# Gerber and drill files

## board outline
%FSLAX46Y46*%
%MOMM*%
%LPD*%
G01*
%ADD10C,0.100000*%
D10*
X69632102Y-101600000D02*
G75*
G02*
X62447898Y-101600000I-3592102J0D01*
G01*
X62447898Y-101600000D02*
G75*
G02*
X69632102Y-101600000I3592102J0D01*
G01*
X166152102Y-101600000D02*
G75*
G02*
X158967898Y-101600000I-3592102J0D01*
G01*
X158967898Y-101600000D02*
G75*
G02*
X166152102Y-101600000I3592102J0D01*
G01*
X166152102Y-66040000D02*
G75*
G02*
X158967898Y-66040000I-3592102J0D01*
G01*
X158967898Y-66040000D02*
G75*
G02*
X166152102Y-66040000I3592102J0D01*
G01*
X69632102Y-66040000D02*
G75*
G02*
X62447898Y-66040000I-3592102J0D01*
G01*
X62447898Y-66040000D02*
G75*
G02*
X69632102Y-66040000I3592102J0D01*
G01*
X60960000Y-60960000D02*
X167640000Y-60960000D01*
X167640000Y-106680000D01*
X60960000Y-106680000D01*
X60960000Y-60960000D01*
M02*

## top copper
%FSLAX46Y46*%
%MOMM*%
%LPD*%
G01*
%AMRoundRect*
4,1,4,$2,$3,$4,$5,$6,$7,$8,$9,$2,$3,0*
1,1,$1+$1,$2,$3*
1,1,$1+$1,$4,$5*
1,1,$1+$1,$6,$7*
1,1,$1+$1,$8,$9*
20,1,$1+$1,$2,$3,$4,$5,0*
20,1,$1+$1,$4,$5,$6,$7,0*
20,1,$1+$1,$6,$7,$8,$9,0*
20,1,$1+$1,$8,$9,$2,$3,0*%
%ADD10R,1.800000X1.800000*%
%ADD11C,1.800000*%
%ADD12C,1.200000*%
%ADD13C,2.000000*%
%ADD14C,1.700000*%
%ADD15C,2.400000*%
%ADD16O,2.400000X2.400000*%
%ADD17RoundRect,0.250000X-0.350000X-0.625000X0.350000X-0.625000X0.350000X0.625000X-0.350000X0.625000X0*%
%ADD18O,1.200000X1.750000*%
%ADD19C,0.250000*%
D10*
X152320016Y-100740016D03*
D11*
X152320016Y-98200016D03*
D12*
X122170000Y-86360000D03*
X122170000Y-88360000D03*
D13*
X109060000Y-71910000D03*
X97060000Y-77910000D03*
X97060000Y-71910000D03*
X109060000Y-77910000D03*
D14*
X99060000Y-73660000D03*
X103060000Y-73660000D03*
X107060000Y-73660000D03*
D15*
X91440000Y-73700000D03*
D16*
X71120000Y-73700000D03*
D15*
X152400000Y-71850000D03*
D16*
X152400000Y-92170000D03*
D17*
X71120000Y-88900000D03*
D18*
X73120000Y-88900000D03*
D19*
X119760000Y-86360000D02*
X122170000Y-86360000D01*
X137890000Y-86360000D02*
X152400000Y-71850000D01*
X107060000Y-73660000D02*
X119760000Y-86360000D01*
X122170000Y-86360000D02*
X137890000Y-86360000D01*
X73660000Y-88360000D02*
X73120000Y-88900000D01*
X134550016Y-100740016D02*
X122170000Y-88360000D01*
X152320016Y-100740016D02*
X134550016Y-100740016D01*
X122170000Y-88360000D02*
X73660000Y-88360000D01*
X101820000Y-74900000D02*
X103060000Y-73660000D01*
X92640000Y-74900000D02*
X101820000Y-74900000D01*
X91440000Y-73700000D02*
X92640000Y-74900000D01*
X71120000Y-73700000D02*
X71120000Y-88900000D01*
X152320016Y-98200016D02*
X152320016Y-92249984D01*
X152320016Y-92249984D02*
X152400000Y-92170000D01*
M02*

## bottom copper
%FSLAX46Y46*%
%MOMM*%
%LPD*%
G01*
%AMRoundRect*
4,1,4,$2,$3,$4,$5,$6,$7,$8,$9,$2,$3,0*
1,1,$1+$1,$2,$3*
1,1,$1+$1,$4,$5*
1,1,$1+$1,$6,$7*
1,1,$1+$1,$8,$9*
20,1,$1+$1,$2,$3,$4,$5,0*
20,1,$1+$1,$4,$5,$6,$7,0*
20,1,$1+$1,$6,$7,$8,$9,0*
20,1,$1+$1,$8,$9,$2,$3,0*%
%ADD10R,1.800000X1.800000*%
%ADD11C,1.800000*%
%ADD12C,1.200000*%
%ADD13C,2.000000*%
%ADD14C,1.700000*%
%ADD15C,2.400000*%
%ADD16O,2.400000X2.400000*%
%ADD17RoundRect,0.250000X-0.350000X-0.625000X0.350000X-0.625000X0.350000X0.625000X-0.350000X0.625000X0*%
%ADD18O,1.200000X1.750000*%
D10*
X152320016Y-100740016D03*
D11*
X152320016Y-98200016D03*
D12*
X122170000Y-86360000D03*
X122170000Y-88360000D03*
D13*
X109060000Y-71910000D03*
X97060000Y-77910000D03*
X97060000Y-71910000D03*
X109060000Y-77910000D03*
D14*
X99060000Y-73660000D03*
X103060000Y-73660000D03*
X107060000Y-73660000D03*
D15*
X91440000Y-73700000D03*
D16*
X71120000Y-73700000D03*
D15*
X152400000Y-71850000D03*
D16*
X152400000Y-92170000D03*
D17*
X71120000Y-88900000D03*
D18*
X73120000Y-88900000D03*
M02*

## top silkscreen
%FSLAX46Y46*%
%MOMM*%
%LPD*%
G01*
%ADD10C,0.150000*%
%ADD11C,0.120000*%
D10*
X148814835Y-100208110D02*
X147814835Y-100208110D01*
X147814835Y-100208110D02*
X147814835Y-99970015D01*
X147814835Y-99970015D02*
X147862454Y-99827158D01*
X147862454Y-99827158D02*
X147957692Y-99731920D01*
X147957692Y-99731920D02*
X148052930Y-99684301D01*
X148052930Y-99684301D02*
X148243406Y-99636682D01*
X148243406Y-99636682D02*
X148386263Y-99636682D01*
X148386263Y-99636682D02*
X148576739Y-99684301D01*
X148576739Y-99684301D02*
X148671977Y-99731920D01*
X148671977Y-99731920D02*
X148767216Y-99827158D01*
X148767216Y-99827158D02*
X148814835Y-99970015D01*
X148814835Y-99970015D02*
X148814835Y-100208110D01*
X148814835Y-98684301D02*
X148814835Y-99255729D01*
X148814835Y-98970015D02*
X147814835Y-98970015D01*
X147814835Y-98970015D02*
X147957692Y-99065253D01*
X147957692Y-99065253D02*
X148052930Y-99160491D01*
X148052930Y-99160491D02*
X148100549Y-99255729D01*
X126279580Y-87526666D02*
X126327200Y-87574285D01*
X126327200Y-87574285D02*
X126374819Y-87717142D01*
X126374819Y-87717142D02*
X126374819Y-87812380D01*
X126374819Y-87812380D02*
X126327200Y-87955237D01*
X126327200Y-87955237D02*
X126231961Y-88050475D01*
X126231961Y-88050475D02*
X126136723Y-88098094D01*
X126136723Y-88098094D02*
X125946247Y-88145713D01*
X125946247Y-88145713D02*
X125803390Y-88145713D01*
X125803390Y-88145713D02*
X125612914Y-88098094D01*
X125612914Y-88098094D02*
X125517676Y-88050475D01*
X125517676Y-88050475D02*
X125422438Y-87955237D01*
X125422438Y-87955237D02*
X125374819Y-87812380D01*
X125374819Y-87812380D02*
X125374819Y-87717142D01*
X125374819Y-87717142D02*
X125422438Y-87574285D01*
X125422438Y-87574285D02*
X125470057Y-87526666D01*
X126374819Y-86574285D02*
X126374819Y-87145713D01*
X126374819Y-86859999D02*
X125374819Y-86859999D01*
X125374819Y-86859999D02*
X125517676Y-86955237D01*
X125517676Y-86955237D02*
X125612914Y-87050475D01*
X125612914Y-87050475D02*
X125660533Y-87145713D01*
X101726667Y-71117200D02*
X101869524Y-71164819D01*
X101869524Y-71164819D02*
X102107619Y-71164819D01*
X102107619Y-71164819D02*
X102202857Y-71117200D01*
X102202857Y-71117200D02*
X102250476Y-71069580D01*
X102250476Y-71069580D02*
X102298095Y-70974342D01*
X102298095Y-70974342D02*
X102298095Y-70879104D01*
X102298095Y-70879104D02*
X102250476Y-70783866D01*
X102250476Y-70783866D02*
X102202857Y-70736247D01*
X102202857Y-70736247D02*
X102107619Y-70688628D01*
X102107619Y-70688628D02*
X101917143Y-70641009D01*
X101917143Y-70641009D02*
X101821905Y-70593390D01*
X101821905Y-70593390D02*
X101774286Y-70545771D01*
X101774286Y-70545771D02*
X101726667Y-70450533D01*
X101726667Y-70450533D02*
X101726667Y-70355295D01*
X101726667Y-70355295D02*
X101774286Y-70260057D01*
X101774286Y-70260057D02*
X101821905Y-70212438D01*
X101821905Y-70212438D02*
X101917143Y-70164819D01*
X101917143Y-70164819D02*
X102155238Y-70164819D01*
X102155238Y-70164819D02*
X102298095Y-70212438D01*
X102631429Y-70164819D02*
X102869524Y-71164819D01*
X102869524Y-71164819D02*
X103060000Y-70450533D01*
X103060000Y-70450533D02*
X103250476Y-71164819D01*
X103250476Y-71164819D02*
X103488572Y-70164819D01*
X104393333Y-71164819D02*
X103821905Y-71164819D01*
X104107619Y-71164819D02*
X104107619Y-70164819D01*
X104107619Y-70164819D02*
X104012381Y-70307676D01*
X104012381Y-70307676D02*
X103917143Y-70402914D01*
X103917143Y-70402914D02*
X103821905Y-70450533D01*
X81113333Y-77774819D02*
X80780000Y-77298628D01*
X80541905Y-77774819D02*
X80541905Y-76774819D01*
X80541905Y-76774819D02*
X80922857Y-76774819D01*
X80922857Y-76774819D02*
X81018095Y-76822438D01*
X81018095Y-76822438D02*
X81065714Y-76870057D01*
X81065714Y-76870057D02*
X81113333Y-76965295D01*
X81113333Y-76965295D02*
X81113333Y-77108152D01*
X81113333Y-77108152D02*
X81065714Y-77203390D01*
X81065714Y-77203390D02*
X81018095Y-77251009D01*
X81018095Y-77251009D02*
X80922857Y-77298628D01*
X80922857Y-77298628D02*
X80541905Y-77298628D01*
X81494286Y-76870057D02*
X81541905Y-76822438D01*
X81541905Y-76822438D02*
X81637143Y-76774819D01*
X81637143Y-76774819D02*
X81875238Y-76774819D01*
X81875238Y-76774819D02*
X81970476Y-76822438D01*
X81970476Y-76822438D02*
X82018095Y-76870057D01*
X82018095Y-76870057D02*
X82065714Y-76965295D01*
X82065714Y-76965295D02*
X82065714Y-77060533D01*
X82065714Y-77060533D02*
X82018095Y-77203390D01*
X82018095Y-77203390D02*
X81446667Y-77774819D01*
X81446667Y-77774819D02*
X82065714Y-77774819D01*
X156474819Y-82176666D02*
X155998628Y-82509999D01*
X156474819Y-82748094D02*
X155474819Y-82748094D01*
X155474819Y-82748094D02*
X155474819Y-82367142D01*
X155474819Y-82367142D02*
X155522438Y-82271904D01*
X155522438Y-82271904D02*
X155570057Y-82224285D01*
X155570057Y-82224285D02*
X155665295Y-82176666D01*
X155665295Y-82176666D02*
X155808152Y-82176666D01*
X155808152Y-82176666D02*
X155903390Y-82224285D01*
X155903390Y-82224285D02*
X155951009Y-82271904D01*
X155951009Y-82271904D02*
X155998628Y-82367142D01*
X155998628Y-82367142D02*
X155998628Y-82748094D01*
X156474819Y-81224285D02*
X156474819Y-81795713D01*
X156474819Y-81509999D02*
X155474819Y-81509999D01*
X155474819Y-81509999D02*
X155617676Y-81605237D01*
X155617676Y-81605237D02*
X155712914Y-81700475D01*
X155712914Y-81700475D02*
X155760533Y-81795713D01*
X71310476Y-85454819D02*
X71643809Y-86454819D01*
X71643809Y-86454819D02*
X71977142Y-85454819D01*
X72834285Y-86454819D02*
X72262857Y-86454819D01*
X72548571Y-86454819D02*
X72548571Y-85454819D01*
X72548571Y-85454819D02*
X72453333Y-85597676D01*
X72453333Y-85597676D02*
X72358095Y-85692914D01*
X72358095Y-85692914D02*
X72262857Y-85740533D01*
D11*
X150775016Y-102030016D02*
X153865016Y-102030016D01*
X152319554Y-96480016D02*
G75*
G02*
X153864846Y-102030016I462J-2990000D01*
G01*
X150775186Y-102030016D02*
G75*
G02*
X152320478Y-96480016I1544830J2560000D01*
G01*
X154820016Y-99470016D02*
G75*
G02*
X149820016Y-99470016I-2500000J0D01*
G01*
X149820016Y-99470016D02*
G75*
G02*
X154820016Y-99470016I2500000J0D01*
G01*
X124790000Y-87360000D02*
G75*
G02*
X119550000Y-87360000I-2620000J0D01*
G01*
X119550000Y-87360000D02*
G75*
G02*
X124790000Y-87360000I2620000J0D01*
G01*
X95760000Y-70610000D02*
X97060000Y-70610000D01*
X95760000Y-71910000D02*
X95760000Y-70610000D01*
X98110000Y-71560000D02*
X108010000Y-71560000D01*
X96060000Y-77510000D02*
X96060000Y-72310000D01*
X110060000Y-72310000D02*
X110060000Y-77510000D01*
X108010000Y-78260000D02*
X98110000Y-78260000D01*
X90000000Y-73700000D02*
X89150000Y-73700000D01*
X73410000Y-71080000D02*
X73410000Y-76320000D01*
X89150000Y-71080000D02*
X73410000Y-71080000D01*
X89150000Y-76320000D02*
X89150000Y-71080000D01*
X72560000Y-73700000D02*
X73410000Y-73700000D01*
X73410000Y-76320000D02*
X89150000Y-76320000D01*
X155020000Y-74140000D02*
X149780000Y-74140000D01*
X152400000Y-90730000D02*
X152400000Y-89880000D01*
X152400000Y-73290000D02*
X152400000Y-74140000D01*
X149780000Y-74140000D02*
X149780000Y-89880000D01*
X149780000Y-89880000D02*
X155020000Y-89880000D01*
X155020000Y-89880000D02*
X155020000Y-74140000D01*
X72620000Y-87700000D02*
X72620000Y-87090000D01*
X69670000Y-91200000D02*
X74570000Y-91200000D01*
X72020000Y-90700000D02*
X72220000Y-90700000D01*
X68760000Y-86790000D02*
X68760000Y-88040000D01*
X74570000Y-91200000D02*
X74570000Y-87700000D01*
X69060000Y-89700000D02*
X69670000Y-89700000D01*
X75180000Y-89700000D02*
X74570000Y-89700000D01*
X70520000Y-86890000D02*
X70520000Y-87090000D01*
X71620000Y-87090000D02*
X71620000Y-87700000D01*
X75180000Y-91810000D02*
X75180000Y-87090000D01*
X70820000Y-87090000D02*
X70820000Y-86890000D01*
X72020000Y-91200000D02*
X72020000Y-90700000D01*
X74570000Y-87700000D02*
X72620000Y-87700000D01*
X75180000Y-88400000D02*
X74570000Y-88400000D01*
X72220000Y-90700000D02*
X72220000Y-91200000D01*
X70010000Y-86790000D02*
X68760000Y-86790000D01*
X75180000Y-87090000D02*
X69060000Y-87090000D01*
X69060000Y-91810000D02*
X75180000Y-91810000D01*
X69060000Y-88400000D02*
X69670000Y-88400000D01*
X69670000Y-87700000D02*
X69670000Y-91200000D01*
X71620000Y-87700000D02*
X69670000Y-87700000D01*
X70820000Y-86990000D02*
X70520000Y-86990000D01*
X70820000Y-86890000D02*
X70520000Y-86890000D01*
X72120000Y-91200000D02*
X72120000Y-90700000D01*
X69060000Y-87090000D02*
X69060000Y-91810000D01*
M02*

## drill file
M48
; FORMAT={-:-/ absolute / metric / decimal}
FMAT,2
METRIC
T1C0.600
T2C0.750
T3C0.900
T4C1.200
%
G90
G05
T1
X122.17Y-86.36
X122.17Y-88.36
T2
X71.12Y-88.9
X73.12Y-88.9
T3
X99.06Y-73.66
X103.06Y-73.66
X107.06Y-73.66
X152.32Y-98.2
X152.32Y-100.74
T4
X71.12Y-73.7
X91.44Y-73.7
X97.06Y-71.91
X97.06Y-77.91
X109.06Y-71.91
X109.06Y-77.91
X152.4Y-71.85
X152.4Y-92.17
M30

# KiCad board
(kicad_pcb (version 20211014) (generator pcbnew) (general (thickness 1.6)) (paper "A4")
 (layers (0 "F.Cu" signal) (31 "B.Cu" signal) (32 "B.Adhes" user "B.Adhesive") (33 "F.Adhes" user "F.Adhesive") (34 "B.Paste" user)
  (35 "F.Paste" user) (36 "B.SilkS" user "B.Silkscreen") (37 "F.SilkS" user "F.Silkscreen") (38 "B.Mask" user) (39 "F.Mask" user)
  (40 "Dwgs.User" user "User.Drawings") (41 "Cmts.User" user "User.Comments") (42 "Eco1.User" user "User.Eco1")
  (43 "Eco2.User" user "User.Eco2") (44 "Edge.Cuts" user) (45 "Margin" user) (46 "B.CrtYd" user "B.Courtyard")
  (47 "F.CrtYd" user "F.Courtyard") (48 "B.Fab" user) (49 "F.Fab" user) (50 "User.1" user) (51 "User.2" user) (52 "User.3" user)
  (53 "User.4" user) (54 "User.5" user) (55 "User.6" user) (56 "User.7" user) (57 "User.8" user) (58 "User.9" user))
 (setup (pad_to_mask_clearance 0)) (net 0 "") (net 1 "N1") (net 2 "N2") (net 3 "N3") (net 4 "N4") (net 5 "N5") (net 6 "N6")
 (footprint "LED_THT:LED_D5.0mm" (layer "F.Cu") (at 152.320016 100.740016 90)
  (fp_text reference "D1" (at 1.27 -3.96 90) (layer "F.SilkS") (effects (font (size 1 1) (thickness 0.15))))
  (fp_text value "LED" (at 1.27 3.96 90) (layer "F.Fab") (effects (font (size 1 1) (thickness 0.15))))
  (fp_line (start -1.29 -1.545) (end -1.29 1.545) (layer "F.SilkS") (width 0.12))
  (fp_arc (start 4.26 -0.000462) (mid 2.072002 2.880433) (end -1.29 1.54483) (layer "F.SilkS") (width 0.12))
  (fp_arc (start -1.29 -1.54483) (mid 2.072002 -2.880433) (end 4.26 0.000462) (layer "F.SilkS") (width 0.12))
  (fp_circle (center 1.27 0) (end 3.77 0) (layer "F.SilkS") (width 0.12) (fill none))
  (pad "1" thru_hole rect (at 0 0 90) (size 1.8 1.8) (drill 0.9) (layers *.Cu *.Mask) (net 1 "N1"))
  (pad "2" thru_hole circle (at 2.54 0 90) (size 1.8 1.8) (drill 0.9) (layers *.Cu *.Mask) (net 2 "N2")))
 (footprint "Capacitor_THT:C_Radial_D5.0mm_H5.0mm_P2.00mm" (layer "F.Cu") (at 122.17 86.36 -90)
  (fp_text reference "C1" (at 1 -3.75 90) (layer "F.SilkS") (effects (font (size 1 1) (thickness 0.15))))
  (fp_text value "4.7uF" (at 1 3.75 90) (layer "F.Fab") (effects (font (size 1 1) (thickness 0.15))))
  (fp_circle (center 1 0) (end 3.62 0) (layer "F.SilkS") (width 0.12) (fill none))
  (pad "1" thru_hole circle (at 0 0 270) (size 1.2 1.2) (drill 0.6) (layers *.Cu *.Mask) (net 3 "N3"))
  (pad "2" thru_hole circle (at 2 0 270) (size 1.2 1.2) (drill 0.6) (layers *.Cu *.Mask) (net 1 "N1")))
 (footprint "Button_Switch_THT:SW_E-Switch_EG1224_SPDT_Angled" (layer "F.Cu") (at 99.06 73.66)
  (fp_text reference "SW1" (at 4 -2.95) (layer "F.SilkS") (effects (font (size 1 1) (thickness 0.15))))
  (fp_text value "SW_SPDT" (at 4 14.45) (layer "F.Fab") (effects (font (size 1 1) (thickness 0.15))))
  (fp_line (start -3.3 -3.05) (end -2 -3.05) (layer "F.SilkS") (width 0.12))
  (fp_line (start -3.3 -1.75) (end -3.3 -3.05) (layer "F.SilkS") (width 0.12))
  (fp_line (start -0.95 -2.1) (end 8.95 -2.1) (layer "F.SilkS") (width 0.12))
  (fp_line (start -3 3.85) (end -3 -1.35) (layer "F.SilkS") (width 0.12))
  (fp_line (start 11 -1.35) (end 11 3.85) (layer "F.SilkS") (width 0.12))
  (fp_line (start 8.95 4.6) (end -0.95 4.6) (layer "F.SilkS") (width 0.12))
  (pad "" thru_hole circle (at 10 -1.75) (size 2 2) (drill 1.2) (layers *.Cu *.Mask))
  (pad "" thru_hole circle (at -2 4.25) (size 2 2) (drill 1.2) (layers *.Cu *.Mask))
  (pad "" thru_hole circle (at -2 -1.75) (size 2 2) (drill 1.2) (layers *.Cu *.Mask))
  (pad "" thru_hole circle (at 10 4.25) (size 2 2) (drill 1.2) (layers *.Cu *.Mask))
  (pad "1" thru_hole circle (at 0 0) (size 1.7 1.7) (drill 0.9) (layers *.Cu *.Mask) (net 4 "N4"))
  (pad "2" thru_hole circle (at 4 0) (size 1.7 1.7) (drill 0.9) (layers *.Cu *.Mask) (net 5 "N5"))
  (pad "3" thru_hole circle (at 8 0) (size 1.7 1.7) (drill 0.9) (layers *.Cu *.Mask) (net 3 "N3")))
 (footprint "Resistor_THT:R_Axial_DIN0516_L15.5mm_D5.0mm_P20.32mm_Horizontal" (layer "F.Cu") (at 91.44 73.7 180)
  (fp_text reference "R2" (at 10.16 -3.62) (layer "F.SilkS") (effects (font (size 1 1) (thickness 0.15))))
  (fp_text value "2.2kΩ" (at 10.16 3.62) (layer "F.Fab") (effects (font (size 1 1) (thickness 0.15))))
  (fp_line (start 1.44 0) (end 2.29 0) (layer "F.SilkS") (width 0.12))
  (fp_line (start 18.03 2.62) (end 18.03 -2.62) (layer "F.SilkS") (width 0.12))
  (fp_line (start 2.29 2.62) (end 18.03 2.62) (layer "F.SilkS") (width 0.12))
  (fp_line (start 2.29 -2.62) (end 2.29 2.62) (layer "F.SilkS") (width 0.12))
  (fp_line (start 18.88 0) (end 18.03 0) (layer "F.SilkS") (width 0.12))
  (fp_line (start 18.03 -2.62) (end 2.29 -2.62) (layer "F.SilkS") (width 0.12))
  (pad "1" thru_hole circle (at 0 0 180) (size 2.4 2.4) (drill 1.2) (layers *.Cu *.Mask) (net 5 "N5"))
  (pad "2" thru_hole oval (at 20.32 0 180) (size 2.4 2.4) (drill 1.2) (layers *.Cu *.Mask) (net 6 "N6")))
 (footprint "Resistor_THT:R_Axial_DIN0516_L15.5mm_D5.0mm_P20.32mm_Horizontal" (layer "F.Cu") (at 152.4 71.85 -90)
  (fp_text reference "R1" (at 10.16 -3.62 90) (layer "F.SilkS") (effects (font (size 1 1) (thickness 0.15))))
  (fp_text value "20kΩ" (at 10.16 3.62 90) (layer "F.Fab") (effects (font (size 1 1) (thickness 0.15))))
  (fp_line (start 2.29 -2.62) (end 2.29 2.62) (layer "F.SilkS") (width 0.12))
  (fp_line (start 18.88 0) (end 18.03 0) (layer "F.SilkS") (width 0.12))
  (fp_line (start 1.44 0) (end 2.29 0) (layer "F.SilkS") (width 0.12))
  (fp_line (start 2.29 2.62) (end 18.03 2.62) (layer "F.SilkS") (width 0.12))
  (fp_line (start 18.03 2.62) (end 18.03 -2.62) (layer "F.SilkS") (width 0.12))
  (fp_line (start 18.03 -2.62) (end 2.29 -2.62) (layer "F.SilkS") (width 0.12))
  (pad "1" thru_hole circle (at 0 0 270) (size 2.4 2.4) (drill 1.2) (layers *.Cu *.Mask) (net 3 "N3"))
  (pad "2" thru_hole oval (at 20.32 0 270) (size 2.4 2.4) (drill 1.2) (layers *.Cu *.Mask) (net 2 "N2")))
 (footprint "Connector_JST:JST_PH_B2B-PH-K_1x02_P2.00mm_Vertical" (layer "F.Cu") (at 71.12 88.9)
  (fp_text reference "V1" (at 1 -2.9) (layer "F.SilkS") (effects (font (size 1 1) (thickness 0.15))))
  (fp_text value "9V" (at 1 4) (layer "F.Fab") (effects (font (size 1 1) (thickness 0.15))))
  (fp_line (start 1.5 -1.2) (end 1.5 -1.81) (layer "F.SilkS") (width 0.12))
  (fp_line (start -1.45 2.3) (end 3.45 2.3) (layer "F.SilkS") (width 0.12))
  (fp_line (start 0.9 1.8) (end 1.1 1.8) (layer "F.SilkS") (width 0.12))
  (fp_line (start -2.36 -2.11) (end -2.36 -0.86) (layer "F.SilkS") (width 0.12))
  (fp_line (start 3.45 2.3) (end 3.45 -1.2) (layer "F.SilkS") (width 0.12))
  (fp_line (start -2.06 0.8) (end -1.45 0.8) (layer "F.SilkS") (width 0.12))
  (fp_line (start 4.06 0.8) (end 3.45 0.8) (layer "F.SilkS") (width 0.12))
  (fp_line (start -0.6 -2.01) (end -0.6 -1.81) (layer "F.SilkS") (width 0.12))
  (fp_line (start 0.5 -1.81) (end 0.5 -1.2) (layer "F.SilkS") (width 0.12))
  (fp_line (start 4.06 2.91) (end 4.06 -1.81) (layer "F.SilkS") (width 0.12))
  (fp_line (start -0.3 -1.81) (end -0.3 -2.01) (layer "F.SilkS") (width 0.12))
  (fp_line (start 0.9 2.3) (end 0.9 1.8) (layer "F.SilkS") (width 0.12))
  (fp_line (start 3.45 -1.2) (end 1.5 -1.2) (layer "F.SilkS") (width 0.12))
  (fp_line (start 4.06 -0.5) (end 3.45 -0.5) (layer "F.SilkS") (width 0.12))
  (fp_line (start 1.1 1.8) (end 1.1 2.3) (layer "F.SilkS") (width 0.12))
  (fp_line (start -1.11 -2.11) (end -2.36 -2.11) (layer "F.SilkS") (width 0.12))
  (fp_line (start 4.06 -1.81) (end -2.06 -1.81) (layer "F.SilkS") (width 0.12))
  (fp_line (start -2.06 2.91) (end 4.06 2.91) (layer "F.SilkS") (width 0.12))
  (fp_line (start -2.06 -0.5) (end -1.45 -0.5) (layer "F.SilkS") (width 0.12))
  (fp_line (start -1.45 -1.2) (end -1.45 2.3) (layer "F.SilkS") (width 0.12))
  (fp_line (start 0.5 -1.2) (end -1.45 -1.2) (layer "F.SilkS") (width 0.12))
  (fp_line (start -0.3 -1.91) (end -0.6 -1.91) (layer "F.SilkS") (width 0.12))
  (fp_line (start -0.3 -2.01) (end -0.6 -2.01) (layer "F.SilkS") (width 0.12))
  (fp_line (start 1 2.3) (end 1 1.8) (layer "F.SilkS") (width 0.12))
  (fp_line (start -2.06 -1.81) (end -2.06 2.91) (layer "F.SilkS") (width 0.12))
  (pad "1" thru_hole roundrect (at 0 0) (size 1.2 1.75) (drill 0.75) (layers *.Cu *.Mask) (roundrect_rratio 0.208333) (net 6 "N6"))
  (pad "2" thru_hole oval (at 2 0) (size 1.2 1.75) (drill 0.75) (layers *.Cu *.Mask) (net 1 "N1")))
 (gr_circle (center 66.04 101.6) (end 68.58 104.14) (layer "Edge.Cuts") (width 0.1) (fill none))
 (gr_circle (center 162.56 101.6) (end 165.1 104.14) (layer "Edge.Cuts") (width 0.1) (fill none))
 (gr_circle (center 162.56 66.04) (end 165.1 68.58) (layer "Edge.Cuts") (width 0.1) (fill none))
 (gr_circle (center 66.04 66.04) (end 68.58 68.58) (layer "Edge.Cuts") (width 0.1) (fill none))
 (gr_rect (start 60.96 60.96) (end 167.64 106.68) (layer "Edge.Cuts") (width 0.1) (fill none))
 (segment (start 119.76 86.36) (end 122.17 86.36) (width 0.25) (layer "F.Cu") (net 3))
 (segment (start 137.89 86.36) (end 152.4 71.85) (width 0.25) (layer "F.Cu") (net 3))
 (segment (start 107.06 73.66) (end 119.76 86.36) (width 0.25) (layer "F.Cu") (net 3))
 (segment (start 122.17 86.36) (end 137.89 86.36) (width 0.25) (layer "F.Cu") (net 3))
 (segment (start 73.66 88.36) (end 73.12 88.9) (width 0.25) (layer "F.Cu") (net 1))
 (segment (start 134.550016 100.740016) (end 122.17 88.36) (width 0.25) (layer "F.Cu") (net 1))
 (segment (start 152.320016 100.740016) (end 134.550016 100.740016) (width 0.25) (layer "F.Cu") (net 1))
 (segment (start 122.17 88.36) (end 73.66 88.36) (width 0.25) (layer "F.Cu") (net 1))
 (segment (start 101.82 74.9) (end 103.06 73.66) (width 0.25) (layer "F.Cu") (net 5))
 (segment (start 92.64 74.9) (end 101.82 74.9) (width 0.25) (layer "F.Cu") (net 5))
 (segment (start 91.44 73.7) (end 92.64 74.9) (width 0.25) (layer "F.Cu") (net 5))
 (segment (start 71.12 73.7) (end 71.12 88.9) (width 0.25) (layer "F.Cu") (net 6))
 (segment (start 152.320016 98.200016) (end 152.320016 92.249984) (width 0.25) (layer "F.Cu") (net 2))
 (segment (start 152.320016 92.249984) (end 152.4 92.17) (width 0.25) (layer "F.Cu") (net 2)))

